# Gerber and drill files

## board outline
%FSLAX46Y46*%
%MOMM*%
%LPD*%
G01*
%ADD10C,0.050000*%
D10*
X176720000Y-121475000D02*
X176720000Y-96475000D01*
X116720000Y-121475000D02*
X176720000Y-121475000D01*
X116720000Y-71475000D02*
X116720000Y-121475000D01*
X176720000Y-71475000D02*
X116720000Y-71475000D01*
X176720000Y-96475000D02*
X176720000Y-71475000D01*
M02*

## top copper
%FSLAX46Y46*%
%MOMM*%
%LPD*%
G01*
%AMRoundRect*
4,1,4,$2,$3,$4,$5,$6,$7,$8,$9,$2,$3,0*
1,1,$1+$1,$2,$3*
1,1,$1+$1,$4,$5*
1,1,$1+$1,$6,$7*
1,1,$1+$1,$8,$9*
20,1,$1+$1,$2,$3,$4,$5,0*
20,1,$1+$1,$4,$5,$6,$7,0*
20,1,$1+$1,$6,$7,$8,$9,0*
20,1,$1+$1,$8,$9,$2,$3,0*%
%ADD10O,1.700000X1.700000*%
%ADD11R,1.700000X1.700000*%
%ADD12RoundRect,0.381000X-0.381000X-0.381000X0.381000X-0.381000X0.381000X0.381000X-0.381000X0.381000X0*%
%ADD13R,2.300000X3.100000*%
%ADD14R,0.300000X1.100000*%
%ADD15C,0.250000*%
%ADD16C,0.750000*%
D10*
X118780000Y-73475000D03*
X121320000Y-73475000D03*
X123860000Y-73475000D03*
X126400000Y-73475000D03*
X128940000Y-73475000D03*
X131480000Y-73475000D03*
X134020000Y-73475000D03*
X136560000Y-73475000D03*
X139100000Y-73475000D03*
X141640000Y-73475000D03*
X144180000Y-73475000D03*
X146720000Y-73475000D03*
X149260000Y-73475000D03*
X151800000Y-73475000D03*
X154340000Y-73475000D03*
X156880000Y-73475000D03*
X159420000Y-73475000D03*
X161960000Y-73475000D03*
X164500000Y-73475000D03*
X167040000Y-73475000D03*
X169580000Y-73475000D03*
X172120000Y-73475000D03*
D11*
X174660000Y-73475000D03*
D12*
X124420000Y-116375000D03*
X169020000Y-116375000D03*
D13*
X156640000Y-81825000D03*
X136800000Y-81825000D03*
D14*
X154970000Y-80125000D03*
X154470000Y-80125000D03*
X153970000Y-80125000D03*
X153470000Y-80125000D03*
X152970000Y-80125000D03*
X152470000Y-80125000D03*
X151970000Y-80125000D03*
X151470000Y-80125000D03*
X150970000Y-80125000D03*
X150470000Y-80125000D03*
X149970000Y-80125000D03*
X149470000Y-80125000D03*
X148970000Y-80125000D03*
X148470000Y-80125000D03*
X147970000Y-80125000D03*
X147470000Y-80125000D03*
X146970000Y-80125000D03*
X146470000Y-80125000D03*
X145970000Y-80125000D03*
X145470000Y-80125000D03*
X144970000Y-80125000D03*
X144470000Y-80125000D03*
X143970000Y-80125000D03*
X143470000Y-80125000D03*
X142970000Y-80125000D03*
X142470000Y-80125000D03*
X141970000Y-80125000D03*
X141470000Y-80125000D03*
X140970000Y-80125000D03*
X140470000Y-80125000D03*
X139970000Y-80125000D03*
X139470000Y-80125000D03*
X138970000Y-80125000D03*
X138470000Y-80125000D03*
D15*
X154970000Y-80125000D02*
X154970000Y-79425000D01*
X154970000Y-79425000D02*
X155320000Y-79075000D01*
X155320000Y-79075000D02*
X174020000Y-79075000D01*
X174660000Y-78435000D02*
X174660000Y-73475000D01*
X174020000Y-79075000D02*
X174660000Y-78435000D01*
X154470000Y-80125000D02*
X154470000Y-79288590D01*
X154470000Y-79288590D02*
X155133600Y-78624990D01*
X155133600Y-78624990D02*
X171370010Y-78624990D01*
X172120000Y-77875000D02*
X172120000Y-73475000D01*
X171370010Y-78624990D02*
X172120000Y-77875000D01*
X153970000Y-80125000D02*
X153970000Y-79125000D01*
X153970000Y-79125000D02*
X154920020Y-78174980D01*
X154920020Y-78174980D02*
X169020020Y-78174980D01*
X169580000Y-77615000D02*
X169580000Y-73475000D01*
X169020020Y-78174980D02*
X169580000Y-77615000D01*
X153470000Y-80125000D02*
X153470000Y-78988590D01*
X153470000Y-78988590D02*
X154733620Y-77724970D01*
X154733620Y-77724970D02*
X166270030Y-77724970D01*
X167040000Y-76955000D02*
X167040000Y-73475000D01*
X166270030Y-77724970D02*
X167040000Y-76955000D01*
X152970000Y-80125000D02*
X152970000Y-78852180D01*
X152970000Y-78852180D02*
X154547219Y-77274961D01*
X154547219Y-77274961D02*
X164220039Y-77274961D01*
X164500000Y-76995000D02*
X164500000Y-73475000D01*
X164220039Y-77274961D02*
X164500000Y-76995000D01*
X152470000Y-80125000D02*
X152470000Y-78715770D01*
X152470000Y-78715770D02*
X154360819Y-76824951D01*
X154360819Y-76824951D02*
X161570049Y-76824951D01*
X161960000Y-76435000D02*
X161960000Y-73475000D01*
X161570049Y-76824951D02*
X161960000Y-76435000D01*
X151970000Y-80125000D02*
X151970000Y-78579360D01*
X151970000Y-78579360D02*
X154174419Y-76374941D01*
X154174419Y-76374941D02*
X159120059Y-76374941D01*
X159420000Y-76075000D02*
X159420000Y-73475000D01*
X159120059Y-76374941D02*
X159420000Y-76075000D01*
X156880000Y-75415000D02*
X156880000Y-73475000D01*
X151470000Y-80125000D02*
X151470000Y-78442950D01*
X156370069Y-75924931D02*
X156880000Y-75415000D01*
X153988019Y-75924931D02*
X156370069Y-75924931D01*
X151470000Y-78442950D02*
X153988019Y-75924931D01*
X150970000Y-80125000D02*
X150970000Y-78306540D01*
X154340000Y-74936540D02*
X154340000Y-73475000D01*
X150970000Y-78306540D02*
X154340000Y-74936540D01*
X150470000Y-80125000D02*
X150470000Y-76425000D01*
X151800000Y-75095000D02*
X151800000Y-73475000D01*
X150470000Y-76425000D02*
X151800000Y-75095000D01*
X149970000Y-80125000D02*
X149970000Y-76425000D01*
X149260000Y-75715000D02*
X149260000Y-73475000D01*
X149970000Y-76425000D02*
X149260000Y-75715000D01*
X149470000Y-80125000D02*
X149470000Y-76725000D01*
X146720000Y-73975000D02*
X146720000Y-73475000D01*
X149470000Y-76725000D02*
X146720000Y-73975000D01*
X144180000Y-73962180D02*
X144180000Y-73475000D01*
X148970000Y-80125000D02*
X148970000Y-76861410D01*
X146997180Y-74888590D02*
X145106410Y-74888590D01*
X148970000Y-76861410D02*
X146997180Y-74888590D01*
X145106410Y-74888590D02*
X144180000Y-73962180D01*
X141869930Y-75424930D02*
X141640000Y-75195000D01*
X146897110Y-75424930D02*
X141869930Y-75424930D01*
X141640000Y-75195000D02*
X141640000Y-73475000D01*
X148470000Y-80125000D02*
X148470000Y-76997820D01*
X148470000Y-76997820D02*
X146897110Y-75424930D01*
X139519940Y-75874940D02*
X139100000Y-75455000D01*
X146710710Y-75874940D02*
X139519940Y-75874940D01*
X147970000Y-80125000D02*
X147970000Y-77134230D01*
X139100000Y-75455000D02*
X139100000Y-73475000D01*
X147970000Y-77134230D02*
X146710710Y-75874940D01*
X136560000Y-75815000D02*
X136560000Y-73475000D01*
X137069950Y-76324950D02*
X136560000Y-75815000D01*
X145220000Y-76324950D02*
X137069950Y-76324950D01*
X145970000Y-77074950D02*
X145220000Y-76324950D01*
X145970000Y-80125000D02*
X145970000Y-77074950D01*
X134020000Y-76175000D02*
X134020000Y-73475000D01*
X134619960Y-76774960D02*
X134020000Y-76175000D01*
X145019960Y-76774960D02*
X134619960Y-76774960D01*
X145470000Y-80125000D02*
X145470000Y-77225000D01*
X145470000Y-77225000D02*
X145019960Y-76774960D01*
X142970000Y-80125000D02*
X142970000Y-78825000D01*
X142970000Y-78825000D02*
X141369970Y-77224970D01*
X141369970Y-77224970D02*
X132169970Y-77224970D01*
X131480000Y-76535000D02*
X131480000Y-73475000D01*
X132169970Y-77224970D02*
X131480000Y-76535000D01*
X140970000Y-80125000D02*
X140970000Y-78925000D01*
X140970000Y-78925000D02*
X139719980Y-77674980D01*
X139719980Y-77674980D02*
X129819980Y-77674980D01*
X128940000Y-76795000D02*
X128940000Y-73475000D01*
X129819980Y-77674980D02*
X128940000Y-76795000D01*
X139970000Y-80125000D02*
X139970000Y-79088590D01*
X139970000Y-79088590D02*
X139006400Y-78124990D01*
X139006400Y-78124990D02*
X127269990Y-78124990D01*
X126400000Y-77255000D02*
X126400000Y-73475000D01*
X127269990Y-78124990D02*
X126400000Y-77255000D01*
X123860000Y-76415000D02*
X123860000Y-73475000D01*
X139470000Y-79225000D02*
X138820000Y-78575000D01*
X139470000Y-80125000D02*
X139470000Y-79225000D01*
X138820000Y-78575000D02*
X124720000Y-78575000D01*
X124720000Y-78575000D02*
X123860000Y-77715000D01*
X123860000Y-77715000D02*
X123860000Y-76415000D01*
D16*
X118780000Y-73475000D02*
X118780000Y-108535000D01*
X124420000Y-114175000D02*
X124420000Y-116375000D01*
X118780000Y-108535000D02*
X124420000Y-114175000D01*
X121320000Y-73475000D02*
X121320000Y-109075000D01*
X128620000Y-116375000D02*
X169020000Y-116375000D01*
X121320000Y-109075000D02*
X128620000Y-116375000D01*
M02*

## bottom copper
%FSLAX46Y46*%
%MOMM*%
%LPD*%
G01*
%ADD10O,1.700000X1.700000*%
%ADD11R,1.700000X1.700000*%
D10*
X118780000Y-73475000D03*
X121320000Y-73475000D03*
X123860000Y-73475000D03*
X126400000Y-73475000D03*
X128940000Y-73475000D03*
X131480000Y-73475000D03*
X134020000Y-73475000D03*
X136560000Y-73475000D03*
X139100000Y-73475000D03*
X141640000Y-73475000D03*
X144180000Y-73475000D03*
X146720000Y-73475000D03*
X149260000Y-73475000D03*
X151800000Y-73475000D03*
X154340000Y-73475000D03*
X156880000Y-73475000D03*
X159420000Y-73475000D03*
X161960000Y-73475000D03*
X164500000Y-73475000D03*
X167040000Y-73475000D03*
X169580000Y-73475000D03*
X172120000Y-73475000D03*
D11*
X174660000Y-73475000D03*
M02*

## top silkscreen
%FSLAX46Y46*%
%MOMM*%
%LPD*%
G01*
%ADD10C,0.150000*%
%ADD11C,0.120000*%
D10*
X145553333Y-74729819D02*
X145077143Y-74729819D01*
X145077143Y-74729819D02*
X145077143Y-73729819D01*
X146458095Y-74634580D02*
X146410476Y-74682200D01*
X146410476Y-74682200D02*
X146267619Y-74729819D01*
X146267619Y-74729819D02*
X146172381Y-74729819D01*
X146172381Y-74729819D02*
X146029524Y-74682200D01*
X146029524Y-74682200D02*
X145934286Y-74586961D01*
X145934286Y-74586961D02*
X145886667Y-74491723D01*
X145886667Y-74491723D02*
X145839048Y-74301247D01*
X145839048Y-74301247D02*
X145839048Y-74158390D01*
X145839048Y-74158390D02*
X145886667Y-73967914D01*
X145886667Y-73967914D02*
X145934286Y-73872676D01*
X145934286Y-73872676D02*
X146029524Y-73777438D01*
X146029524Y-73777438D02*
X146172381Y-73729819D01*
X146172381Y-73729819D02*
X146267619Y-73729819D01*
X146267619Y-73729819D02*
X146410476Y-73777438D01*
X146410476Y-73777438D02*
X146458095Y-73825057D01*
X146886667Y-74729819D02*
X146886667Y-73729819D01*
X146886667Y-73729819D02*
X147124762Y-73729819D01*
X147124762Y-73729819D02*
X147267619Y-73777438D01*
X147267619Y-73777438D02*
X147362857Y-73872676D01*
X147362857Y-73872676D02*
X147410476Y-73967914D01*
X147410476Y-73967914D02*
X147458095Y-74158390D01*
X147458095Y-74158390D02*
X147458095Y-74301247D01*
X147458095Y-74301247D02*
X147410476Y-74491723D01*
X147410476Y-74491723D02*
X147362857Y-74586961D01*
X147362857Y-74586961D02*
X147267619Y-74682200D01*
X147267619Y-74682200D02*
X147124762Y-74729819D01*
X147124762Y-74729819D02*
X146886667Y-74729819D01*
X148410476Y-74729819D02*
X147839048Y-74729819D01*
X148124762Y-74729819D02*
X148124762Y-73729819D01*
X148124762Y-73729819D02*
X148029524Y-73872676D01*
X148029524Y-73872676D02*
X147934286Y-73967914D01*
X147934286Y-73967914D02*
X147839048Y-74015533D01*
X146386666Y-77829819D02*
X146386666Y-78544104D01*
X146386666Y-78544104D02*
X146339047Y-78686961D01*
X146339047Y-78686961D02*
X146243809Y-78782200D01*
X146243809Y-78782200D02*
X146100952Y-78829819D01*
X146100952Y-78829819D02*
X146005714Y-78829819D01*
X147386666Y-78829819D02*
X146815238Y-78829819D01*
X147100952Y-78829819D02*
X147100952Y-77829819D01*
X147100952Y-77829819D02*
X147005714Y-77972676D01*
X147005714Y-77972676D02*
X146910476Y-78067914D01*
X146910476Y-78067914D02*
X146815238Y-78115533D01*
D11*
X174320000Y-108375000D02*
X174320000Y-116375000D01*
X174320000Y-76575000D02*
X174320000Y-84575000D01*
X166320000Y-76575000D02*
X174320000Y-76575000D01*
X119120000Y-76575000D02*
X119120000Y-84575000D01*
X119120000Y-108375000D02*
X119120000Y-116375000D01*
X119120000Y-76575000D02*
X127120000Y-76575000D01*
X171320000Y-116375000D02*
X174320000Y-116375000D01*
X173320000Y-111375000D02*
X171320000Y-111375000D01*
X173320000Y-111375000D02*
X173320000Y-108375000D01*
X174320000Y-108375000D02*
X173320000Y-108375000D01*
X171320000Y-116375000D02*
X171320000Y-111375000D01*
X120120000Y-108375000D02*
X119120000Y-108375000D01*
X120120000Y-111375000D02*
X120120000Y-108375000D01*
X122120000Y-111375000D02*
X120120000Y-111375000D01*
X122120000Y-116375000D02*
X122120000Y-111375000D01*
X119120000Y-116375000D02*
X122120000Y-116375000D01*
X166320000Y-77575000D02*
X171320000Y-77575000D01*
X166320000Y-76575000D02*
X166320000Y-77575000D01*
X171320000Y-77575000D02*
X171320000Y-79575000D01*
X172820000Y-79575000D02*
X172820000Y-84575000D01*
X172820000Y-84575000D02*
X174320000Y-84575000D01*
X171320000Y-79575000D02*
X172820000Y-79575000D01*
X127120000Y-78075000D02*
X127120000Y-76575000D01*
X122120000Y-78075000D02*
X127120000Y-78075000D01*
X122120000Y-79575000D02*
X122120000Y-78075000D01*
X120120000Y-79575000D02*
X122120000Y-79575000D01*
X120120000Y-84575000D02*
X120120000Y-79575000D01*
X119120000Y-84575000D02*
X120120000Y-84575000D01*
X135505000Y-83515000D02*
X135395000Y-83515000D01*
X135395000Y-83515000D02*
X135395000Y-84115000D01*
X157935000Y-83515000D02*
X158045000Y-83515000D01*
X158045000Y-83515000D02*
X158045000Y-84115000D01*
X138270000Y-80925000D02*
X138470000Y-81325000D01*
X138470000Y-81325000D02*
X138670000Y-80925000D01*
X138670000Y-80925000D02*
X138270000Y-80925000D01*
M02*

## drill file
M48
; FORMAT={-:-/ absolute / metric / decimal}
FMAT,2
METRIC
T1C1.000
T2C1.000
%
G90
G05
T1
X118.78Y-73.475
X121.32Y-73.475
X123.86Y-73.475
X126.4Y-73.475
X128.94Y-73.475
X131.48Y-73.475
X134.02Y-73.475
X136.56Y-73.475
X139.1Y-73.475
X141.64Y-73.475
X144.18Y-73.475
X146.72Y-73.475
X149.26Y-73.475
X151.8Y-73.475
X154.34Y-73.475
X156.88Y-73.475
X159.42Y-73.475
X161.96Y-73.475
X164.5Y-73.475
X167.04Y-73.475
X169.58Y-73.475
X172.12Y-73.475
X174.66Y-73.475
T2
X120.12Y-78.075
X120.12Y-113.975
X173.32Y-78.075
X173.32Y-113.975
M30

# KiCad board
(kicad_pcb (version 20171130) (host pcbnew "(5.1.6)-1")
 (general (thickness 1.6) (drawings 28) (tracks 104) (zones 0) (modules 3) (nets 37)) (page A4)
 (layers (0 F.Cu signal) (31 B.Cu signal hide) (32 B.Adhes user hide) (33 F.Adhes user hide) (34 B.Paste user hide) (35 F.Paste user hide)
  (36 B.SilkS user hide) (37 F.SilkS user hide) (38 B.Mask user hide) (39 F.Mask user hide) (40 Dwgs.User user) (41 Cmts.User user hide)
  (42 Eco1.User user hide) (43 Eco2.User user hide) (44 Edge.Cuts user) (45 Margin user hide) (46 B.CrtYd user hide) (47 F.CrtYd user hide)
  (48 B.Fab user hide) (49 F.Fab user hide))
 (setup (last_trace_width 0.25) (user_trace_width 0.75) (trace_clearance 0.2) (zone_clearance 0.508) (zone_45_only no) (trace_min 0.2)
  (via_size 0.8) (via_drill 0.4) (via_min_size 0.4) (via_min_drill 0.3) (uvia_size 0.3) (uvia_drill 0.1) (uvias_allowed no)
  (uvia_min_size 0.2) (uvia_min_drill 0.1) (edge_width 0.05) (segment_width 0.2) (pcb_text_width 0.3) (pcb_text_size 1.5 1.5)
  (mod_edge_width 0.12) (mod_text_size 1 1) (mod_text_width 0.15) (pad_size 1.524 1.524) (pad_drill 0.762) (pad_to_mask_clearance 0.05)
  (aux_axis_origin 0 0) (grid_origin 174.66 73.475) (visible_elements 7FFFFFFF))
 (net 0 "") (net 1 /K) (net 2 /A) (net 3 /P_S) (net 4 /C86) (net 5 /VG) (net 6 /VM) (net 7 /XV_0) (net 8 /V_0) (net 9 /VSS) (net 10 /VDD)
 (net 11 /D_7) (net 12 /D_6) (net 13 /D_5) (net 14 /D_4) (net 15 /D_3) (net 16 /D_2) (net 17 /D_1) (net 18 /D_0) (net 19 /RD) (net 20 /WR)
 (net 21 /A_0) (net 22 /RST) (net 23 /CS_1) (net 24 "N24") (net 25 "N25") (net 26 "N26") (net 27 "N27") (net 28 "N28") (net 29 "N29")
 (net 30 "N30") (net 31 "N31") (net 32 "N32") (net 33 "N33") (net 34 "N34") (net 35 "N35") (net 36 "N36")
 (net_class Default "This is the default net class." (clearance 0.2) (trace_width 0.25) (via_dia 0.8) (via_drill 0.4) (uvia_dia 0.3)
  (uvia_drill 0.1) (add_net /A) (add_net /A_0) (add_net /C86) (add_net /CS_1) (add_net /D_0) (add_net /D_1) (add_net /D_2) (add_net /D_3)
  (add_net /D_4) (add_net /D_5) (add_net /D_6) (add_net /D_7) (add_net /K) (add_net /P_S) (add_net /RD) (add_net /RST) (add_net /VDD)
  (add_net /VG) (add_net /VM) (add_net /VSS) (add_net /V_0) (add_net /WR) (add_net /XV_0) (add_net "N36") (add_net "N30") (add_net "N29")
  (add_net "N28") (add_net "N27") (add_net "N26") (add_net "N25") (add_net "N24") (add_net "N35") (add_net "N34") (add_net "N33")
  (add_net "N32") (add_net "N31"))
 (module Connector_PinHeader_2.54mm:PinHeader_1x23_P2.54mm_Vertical (layer B.Cu) (at 174.66 73.475 90)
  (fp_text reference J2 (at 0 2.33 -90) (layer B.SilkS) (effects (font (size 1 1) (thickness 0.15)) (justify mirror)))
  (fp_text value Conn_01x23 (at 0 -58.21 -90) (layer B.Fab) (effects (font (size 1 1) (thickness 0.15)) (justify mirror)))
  (pad 23 thru_hole oval (at 0 -55.88 90) (size 1.7 1.7) (drill 1) (layers *.Cu *.Mask) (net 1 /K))
  (pad 22 thru_hole oval (at 0 -53.34 90) (size 1.7 1.7) (drill 1) (layers *.Cu *.Mask) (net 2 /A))
  (pad 21 thru_hole oval (at 0 -50.8 90) (size 1.7 1.7) (drill 1) (layers *.Cu *.Mask) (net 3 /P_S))
  (pad 20 thru_hole oval (at 0 -48.26 90) (size 1.7 1.7) (drill 1) (layers *.Cu *.Mask) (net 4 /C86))
  (pad 19 thru_hole oval (at 0 -45.72 90) (size 1.7 1.7) (drill 1) (layers *.Cu *.Mask) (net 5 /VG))
  (pad 18 thru_hole oval (at 0 -43.18 90) (size 1.7 1.7) (drill 1) (layers *.Cu *.Mask) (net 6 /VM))
  (pad 17 thru_hole oval (at 0 -40.64 90) (size 1.7 1.7) (drill 1) (layers *.Cu *.Mask) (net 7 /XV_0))
  (pad 16 thru_hole oval (at 0 -38.1 90) (size 1.7 1.7) (drill 1) (layers *.Cu *.Mask) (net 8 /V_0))
  (pad 15 thru_hole oval (at 0 -35.56 90) (size 1.7 1.7) (drill 1) (layers *.Cu *.Mask) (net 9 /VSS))
  (pad 14 thru_hole oval (at 0 -33.02 90) (size 1.7 1.7) (drill 1) (layers *.Cu *.Mask) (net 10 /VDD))
  (pad 13 thru_hole oval (at 0 -30.48 90) (size 1.7 1.7) (drill 1) (layers *.Cu *.Mask) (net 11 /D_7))
  (pad 12 thru_hole oval (at 0 -27.94 90) (size 1.7 1.7) (drill 1) (layers *.Cu *.Mask) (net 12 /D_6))
  (pad 11 thru_hole oval (at 0 -25.4 90) (size 1.7 1.7) (drill 1) (layers *.Cu *.Mask) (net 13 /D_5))
  (pad 10 thru_hole oval (at 0 -22.86 90) (size 1.7 1.7) (drill 1) (layers *.Cu *.Mask) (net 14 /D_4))
  (pad 9 thru_hole oval (at 0 -20.32 90) (size 1.7 1.7) (drill 1) (layers *.Cu *.Mask) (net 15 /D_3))
  (pad 8 thru_hole oval (at 0 -17.78 90) (size 1.7 1.7) (drill 1) (layers *.Cu *.Mask) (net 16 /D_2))
  (pad 7 thru_hole oval (at 0 -15.24 90) (size 1.7 1.7) (drill 1) (layers *.Cu *.Mask) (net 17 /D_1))
  (pad 6 thru_hole oval (at 0 -12.7 90) (size 1.7 1.7) (drill 1) (layers *.Cu *.Mask) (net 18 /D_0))
  (pad 5 thru_hole oval (at 0 -10.16 90) (size 1.7 1.7) (drill 1) (layers *.Cu *.Mask) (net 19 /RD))
  (pad 4 thru_hole oval (at 0 -7.62 90) (size 1.7 1.7) (drill 1) (layers *.Cu *.Mask) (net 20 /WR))
  (pad 3 thru_hole oval (at 0 -5.08 90) (size 1.7 1.7) (drill 1) (layers *.Cu *.Mask) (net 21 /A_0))
  (pad 2 thru_hole oval (at 0 -2.54 90) (size 1.7 1.7) (drill 1) (layers *.Cu *.Mask) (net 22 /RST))
  (pad 1 thru_hole rect (at 0 0 90) (size 1.7 1.7) (drill 1) (layers *.Cu *.Mask) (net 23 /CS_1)))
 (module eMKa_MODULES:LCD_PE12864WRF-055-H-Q (layer F.Cu) (at 146.72 96.475)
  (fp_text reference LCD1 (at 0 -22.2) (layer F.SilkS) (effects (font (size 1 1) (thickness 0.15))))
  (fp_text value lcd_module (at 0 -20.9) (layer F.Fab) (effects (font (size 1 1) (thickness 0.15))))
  (fp_line (start 27.6 11.9) (end 27.6 19.9) (layer F.SilkS) (width 0.12))
  (fp_line (start 27.6 -19.9) (end 27.6 -11.9) (layer F.SilkS) (width 0.12))
  (fp_line (start 19.6 -19.9) (end 27.6 -19.9) (layer F.SilkS) (width 0.12))
  (fp_line (start -27.6 -19.9) (end -27.6 -11.9) (layer F.SilkS) (width 0.12))
  (fp_line (start -27.6 11.9) (end -27.6 19.9) (layer F.SilkS) (width 0.12))
  (fp_line (start -27.6 -19.9) (end -19.6 -19.9) (layer F.SilkS) (width 0.12))
  (fp_line (start 24.6 19.9) (end 27.6 19.9) (layer F.SilkS) (width 0.12))
  (fp_line (start 26.6 14.9) (end 24.6 14.9) (layer F.SilkS) (width 0.12))
  (fp_line (start 26.6 14.9) (end 26.6 11.9) (layer F.SilkS) (width 0.12))
  (fp_line (start 27.6 11.9) (end 26.6 11.9) (layer F.SilkS) (width 0.12))
  (fp_line (start 24.6 19.9) (end 24.6 14.9) (layer F.SilkS) (width 0.12))
  (fp_line (start -26.6 11.9) (end -27.6 11.9) (layer F.SilkS) (width 0.12))
  (fp_line (start -26.6 14.9) (end -26.6 11.9) (layer F.SilkS) (width 0.12))
  (fp_line (start -24.6 14.9) (end -26.6 14.9) (layer F.SilkS) (width 0.12))
  (fp_line (start -24.6 19.9) (end -24.6 14.9) (layer F.SilkS) (width 0.12))
  (fp_line (start -27.6 19.9) (end -24.6 19.9) (layer F.SilkS) (width 0.12))
  (fp_line (start 19.6 -18.9) (end 24.6 -18.9) (layer F.SilkS) (width 0.12))
  (fp_line (start 19.6 -19.9) (end 19.6 -18.9) (layer F.SilkS) (width 0.12))
  (fp_line (start 24.6 -18.9) (end 24.6 -16.9) (layer F.SilkS) (width 0.12))
  (fp_line (start 26.1 -16.9) (end 26.1 -11.9) (layer F.SilkS) (width 0.12))
  (fp_line (start 26.1 -11.9) (end 27.6 -11.9) (layer F.SilkS) (width 0.12))
  (fp_line (start 24.6 -16.9) (end 26.1 -16.9) (layer F.SilkS) (width 0.12))
  (fp_line (start -19.6 -18.4) (end -19.6 -19.9) (layer F.SilkS) (width 0.12))
  (fp_line (start -24.6 -18.4) (end -19.6 -18.4) (layer F.SilkS) (width 0.12))
  (fp_line (start -24.6 -16.9) (end -24.6 -18.4) (layer F.SilkS) (width 0.12))
  (fp_line (start -26.6 -16.9) (end -24.6 -16.9) (layer F.SilkS) (width 0.12))
  (fp_line (start -26.6 -11.9) (end -26.6 -16.9) (layer F.SilkS) (width 0.12))
  (fp_line (start -27.6 -11.9) (end -26.6 -11.9) (layer F.SilkS) (width 0.12))
  (pad 1 smd roundrect (at -22.3 19.9) (size 1.524 1.524) (layers F.Cu F.Paste F.Mask) (roundrect_rratio 0.25) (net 1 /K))
  (pad 2 smd roundrect (at 22.3 19.9) (size 1.524 1.524) (layers F.Cu F.Paste F.Mask) (roundrect_rratio 0.25) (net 2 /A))
  (pad "" np_thru_hole circle (at -26.6 17.5) (size 1 1) (drill 1) (layers *.Cu *.Mask))
  (pad "" np_thru_hole circle (at 26.6 17.5) (size 1 1) (drill 1) (layers *.Cu *.Mask))
  (pad "" np_thru_hole circle (at 26.6 -18.4) (size 1 1) (drill 1) (layers *.Cu *.Mask))
  (pad "" np_thru_hole circle (at -26.6 -18.4) (size 1 1) (drill 1) (layers *.Cu *.Mask)))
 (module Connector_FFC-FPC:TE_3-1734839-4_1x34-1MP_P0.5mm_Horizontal (layer F.Cu) (at 146.72 81.475)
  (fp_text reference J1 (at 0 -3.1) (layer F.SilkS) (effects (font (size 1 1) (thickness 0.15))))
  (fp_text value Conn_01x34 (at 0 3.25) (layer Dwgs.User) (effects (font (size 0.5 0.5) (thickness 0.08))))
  (fp_line (start -11.215 2.04) (end -11.325 2.04) (layer F.SilkS) (width 0.12))
  (fp_line (start -11.325 2.04) (end -11.325 2.64) (layer F.SilkS) (width 0.12))
  (fp_line (start 11.215 2.04) (end 11.325 2.04) (layer F.SilkS) (width 0.12))
  (fp_line (start 11.325 2.04) (end 11.325 2.64) (layer F.SilkS) (width 0.12))
  (fp_line (start -8.45 -0.55) (end -8.25 -0.15) (layer F.SilkS) (width 0.12))
  (fp_line (start -8.25 -0.15) (end -8.05 -0.55) (layer F.SilkS) (width 0.12))
  (fp_line (start -8.05 -0.55) (end -8.45 -0.55) (layer F.SilkS) (width 0.12))
  (pad MP smd rect (at 9.92 0.35) (size 2.3 3.1) (layers F.Cu F.Paste F.Mask))
  (pad MP smd rect (at -9.92 0.35) (size 2.3 3.1) (layers F.Cu F.Paste F.Mask))
  (pad 34 smd rect (at 8.25 -1.35) (size 0.3 1.1) (layers F.Cu F.Paste F.Mask) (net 23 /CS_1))
  (pad 33 smd rect (at 7.75 -1.35) (size 0.3 1.1) (layers F.Cu F.Paste F.Mask) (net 22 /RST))
  (pad 32 smd rect (at 7.25 -1.35) (size 0.3 1.1) (layers F.Cu F.Paste F.Mask) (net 21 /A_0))
  (pad 31 smd rect (at 6.75 -1.35) (size 0.3 1.1) (layers F.Cu F.Paste F.Mask) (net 20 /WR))
  (pad 30 smd rect (at 6.25 -1.35) (size 0.3 1.1) (layers F.Cu F.Paste F.Mask) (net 19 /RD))
  (pad 29 smd rect (at 5.75 -1.35) (size 0.3 1.1) (layers F.Cu F.Paste F.Mask) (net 18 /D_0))
  (pad 28 smd rect (at 5.25 -1.35) (size 0.3 1.1) (layers F.Cu F.Paste F.Mask) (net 17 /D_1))
  (pad 27 smd rect (at 4.75 -1.35) (size 0.3 1.1) (layers F.Cu F.Paste F.Mask) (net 16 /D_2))
  (pad 26 smd rect (at 4.25 -1.35) (size 0.3 1.1) (layers F.Cu F.Paste F.Mask) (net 15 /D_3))
  (pad 25 smd rect (at 3.75 -1.35) (size 0.3 1.1) (layers F.Cu F.Paste F.Mask) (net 14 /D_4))
  (pad 24 smd rect (at 3.25 -1.35) (size 0.3 1.1) (layers F.Cu F.Paste F.Mask) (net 13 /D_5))
  (pad 23 smd rect (at 2.75 -1.35) (size 0.3 1.1) (layers F.Cu F.Paste F.Mask) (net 12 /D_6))
  (pad 22 smd rect (at 2.25 -1.35) (size 0.3 1.1) (layers F.Cu F.Paste F.Mask) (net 11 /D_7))
  (pad 21 smd rect (at 1.75 -1.35) (size 0.3 1.1) (layers F.Cu F.Paste F.Mask) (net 10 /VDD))
  (pad 20 smd rect (at 1.25 -1.35) (size 0.3 1.1) (layers F.Cu F.Paste F.Mask) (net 9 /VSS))
  (pad 19 smd rect (at 0.75 -1.35) (size 0.3 1.1) (layers F.Cu F.Paste F.Mask) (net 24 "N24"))
  (pad 18 smd rect (at 0.25 -1.35) (size 0.3 1.1) (layers F.Cu F.Paste F.Mask) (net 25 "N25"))
  (pad 17 smd rect (at -0.25 -1.35) (size 0.3 1.1) (layers F.Cu F.Paste F.Mask) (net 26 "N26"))
  (pad 16 smd rect (at -0.75 -1.35) (size 0.3 1.1) (layers F.Cu F.Paste F.Mask) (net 8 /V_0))
  (pad 15 smd rect (at -1.25 -1.35) (size 0.3 1.1) (layers F.Cu F.Paste F.Mask) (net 7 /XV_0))
  (pad 14 smd rect (at -1.75 -1.35) (size 0.3 1.1) (layers F.Cu F.Paste F.Mask) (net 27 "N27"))
  (pad 13 smd rect (at -2.25 -1.35) (size 0.3 1.1) (layers F.Cu F.Paste F.Mask) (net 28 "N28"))
  (pad 12 smd rect (at -2.75 -1.35) (size 0.3 1.1) (layers F.Cu F.Paste F.Mask) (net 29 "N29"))
  (pad 11 smd rect (at -3.25 -1.35) (size 0.3 1.1) (layers F.Cu F.Paste F.Mask) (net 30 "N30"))
  (pad 10 smd rect (at -3.75 -1.35) (size 0.3 1.1) (layers F.Cu F.Paste F.Mask) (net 6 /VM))
  (pad 9 smd rect (at -4.25 -1.35) (size 0.3 1.1) (layers F.Cu F.Paste F.Mask) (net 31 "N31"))
  (pad 8 smd rect (at -4.75 -1.35) (size 0.3 1.1) (layers F.Cu F.Paste F.Mask) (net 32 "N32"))
  (pad 7 smd rect (at -5.25 -1.35) (size 0.3 1.1) (layers F.Cu F.Paste F.Mask) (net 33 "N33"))
  (pad 6 smd rect (at -5.75 -1.35) (size 0.3 1.1) (layers F.Cu F.Paste F.Mask) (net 5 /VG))
  (pad 5 smd rect (at -6.25 -1.35) (size 0.3 1.1) (layers F.Cu F.Paste F.Mask) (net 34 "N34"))
  (pad 4 smd rect (at -6.75 -1.35) (size 0.3 1.1) (layers F.Cu F.Paste F.Mask) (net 4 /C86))
  (pad 3 smd rect (at -7.25 -1.35) (size 0.3 1.1) (layers F.Cu F.Paste F.Mask) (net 3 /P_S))
  (pad 2 smd rect (at -7.75 -1.35) (size 0.3 1.1) (layers F.Cu F.Paste F.Mask) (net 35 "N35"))
  (pad 1 smd rect (at -8.25 -1.35) (size 0.3 1.1) (layers F.Cu F.Paste F.Mask) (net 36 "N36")))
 (gr_line (start 176.72 121.475) (end 176.72 96.475) (layer Edge.Cuts) (width 0.05))
 (gr_line (start 116.72 121.475) (end 176.72 121.475) (layer Edge.Cuts) (width 0.05))
 (gr_line (start 116.72 71.475) (end 116.72 121.475) (layer Edge.Cuts) (width 0.05))
 (gr_line (start 176.72 71.475) (end 116.72 71.475) (layer Edge.Cuts) (width 0.05))
 (gr_line (start 176.72 96.475) (end 176.72 71.475) (layer Edge.Cuts) (width 0.05))
 (segment (start 154.97 80.125) (end 154.97 79.425) (width 0.25) (layer F.Cu) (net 23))
 (segment (start 154.97 79.425) (end 155.32 79.075) (width 0.25) (layer F.Cu) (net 23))
 (segment (start 155.32 79.075) (end 174.02 79.075) (width 0.25) (layer F.Cu) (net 23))
 (segment (start 174.66 78.435) (end 174.66 73.475) (width 0.25) (layer F.Cu) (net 23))
 (segment (start 174.02 79.075) (end 174.66 78.435) (width 0.25) (layer F.Cu) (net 23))
 (segment (start 154.47 80.125) (end 154.47 79.28859) (width 0.25) (layer F.Cu) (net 22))
 (segment (start 154.47 79.28859) (end 155.1336 78.62499) (width 0.25) (layer F.Cu) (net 22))
 (segment (start 155.1336 78.62499) (end 171.37001 78.62499) (width 0.25) (layer F.Cu) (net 22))
 (segment (start 172.12 77.875) (end 172.12 73.475) (width 0.25) (layer F.Cu) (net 22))
 (segment (start 171.37001 78.62499) (end 172.12 77.875) (width 0.25) (layer F.Cu) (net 22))
 (segment (start 153.97 80.125) (end 153.97 79.125) (width 0.25) (layer F.Cu) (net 21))
 (segment (start 153.97 79.125) (end 154.92002 78.17498) (width 0.25) (layer F.Cu) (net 21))
 (segment (start 154.92002 78.17498) (end 169.02002 78.17498) (width 0.25) (layer F.Cu) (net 21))
 (segment (start 169.58 77.615) (end 169.58 73.475) (width 0.25) (layer F.Cu) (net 21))
 (segment (start 169.02002 78.17498) (end 169.58 77.615) (width 0.25) (layer F.Cu) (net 21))
 (segment (start 153.47 80.125) (end 153.47 78.98859) (width 0.25) (layer F.Cu) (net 20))
 (segment (start 153.47 78.98859) (end 154.73362 77.72497) (width 0.25) (layer F.Cu) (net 20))
 (segment (start 154.73362 77.72497) (end 166.27003 77.72497) (width 0.25) (layer F.Cu) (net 20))
 (segment (start 167.04 76.955) (end 167.04 73.475) (width 0.25) (layer F.Cu) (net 20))
 (segment (start 166.27003 77.72497) (end 167.04 76.955) (width 0.25) (layer F.Cu) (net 20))
 (segment (start 152.97 80.125) (end 152.97 78.85218) (width 0.25) (layer F.Cu) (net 19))
 (segment (start 152.97 78.85218) (end 154.547219 77.274961) (width 0.25) (layer F.Cu) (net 19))
 (segment (start 154.547219 77.274961) (end 164.220039 77.274961) (width 0.25) (layer F.Cu) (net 19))
 (segment (start 164.5 76.995) (end 164.5 73.475) (width 0.25) (layer F.Cu) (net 19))
 (segment (start 164.220039 77.274961) (end 164.5 76.995) (width 0.25) (layer F.Cu) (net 19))
 (segment (start 152.47 80.125) (end 152.47 78.71577) (width 0.25) (layer F.Cu) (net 18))
 (segment (start 152.47 78.71577) (end 154.360819 76.824951) (width 0.25) (layer F.Cu) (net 18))
 (segment (start 154.360819 76.824951) (end 161.570049 76.824951) (width 0.25) (layer F.Cu) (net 18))
 (segment (start 161.96 76.435) (end 161.96 73.475) (width 0.25) (layer F.Cu) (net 18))
 (segment (start 161.570049 76.824951) (end 161.96 76.435) (width 0.25) (layer F.Cu) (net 18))
 (segment (start 151.97 80.125) (end 151.97 78.57936) (width 0.25) (layer F.Cu) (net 17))
 (segment (start 151.97 78.57936) (end 154.174419 76.374941) (width 0.25) (layer F.Cu) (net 17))
 (segment (start 154.174419 76.374941) (end 159.120059 76.374941) (width 0.25) (layer F.Cu) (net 17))
 (segment (start 159.42 76.075) (end 159.42 73.475) (width 0.25) (layer F.Cu) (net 17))
 (segment (start 159.120059 76.374941) (end 159.42 76.075) (width 0.25) (layer F.Cu) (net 17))
 (segment (start 156.88 75.415) (end 156.88 73.475) (width 0.25) (layer F.Cu) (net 16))
 (segment (start 151.47 80.125) (end 151.47 78.44295) (width 0.25) (layer F.Cu) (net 16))
 (segment (start 156.370069 75.924931) (end 156.88 75.415) (width 0.25) (layer F.Cu) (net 16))
 (segment (start 153.988019 75.924931) (end 156.370069 75.924931) (width 0.25) (layer F.Cu) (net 16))
 (segment (start 151.47 78.44295) (end 153.988019 75.924931) (width 0.25) (layer F.Cu) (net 16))
 (segment (start 150.97 80.125) (end 150.97 78.30654) (width 0.25) (layer F.Cu) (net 15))
 (segment (start 154.34 74.93654) (end 154.34 73.475) (width 0.25) (layer F.Cu) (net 15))
 (segment (start 150.97 78.30654) (end 154.34 74.93654) (width 0.25) (layer F.Cu) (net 15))
 (segment (start 150.47 80.125) (end 150.47 76.425) (width 0.25) (layer F.Cu) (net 14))
 (segment (start 151.8 75.095) (end 151.8 73.475) (width 0.25) (layer F.Cu) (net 14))
 (segment (start 150.47 76.425) (end 151.8 75.095) (width 0.25) (layer F.Cu) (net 14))
 (segment (start 149.97 80.125) (end 149.97 76.425) (width 0.25) (layer F.Cu) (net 13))
 (segment (start 149.26 75.715) (end 149.26 73.475) (width 0.25) (layer F.Cu) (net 13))
 (segment (start 149.97 76.425) (end 149.26 75.715) (width 0.25) (layer F.Cu) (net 13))
 (segment (start 149.47 80.125) (end 149.47 76.725) (width 0.25) (layer F.Cu) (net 12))
 (segment (start 146.72 73.975) (end 146.72 73.475) (width 0.25) (layer F.Cu) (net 12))
 (segment (start 149.47 76.725) (end 146.72 73.975) (width 0.25) (layer F.Cu) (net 12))
 (segment (start 144.18 73.96218) (end 144.18 73.475) (width 0.25) (layer F.Cu) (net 11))
 (segment (start 148.97 80.125) (end 148.97 76.86141) (width 0.25) (layer F.Cu) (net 11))
 (segment (start 146.99718 74.88859) (end 145.10641 74.88859) (width 0.25) (layer F.Cu) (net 11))
 (segment (start 148.97 76.86141) (end 146.99718 74.88859) (width 0.25) (layer F.Cu) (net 11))
 (segment (start 145.10641 74.88859) (end 144.18 73.96218) (width 0.25) (layer F.Cu) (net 11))
 (segment (start 141.86993 75.42493) (end 141.64 75.195) (width 0.25) (layer F.Cu) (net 10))
 (segment (start 146.89711 75.42493) (end 141.86993 75.42493) (width 0.25) (layer F.Cu) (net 10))
 (segment (start 141.64 75.195) (end 141.64 73.475) (width 0.25) (layer F.Cu) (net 10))
 (segment (start 148.47 80.125) (end 148.47 76.99782) (width 0.25) (layer F.Cu) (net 10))
 (segment (start 148.47 76.99782) (end 146.89711 75.42493) (width 0.25) (layer F.Cu) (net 10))
 (segment (start 139.51994 75.87494) (end 139.1 75.455) (width 0.25) (layer F.Cu) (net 9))
 (segment (start 146.71071 75.87494) (end 139.51994 75.87494) (width 0.25) (layer F.Cu) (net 9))
 (segment (start 147.97 80.125) (end 147.97 77.13423) (width 0.25) (layer F.Cu) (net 9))
 (segment (start 139.1 75.455) (end 139.1 73.475) (width 0.25) (layer F.Cu) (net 9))
 (segment (start 147.97 77.13423) (end 146.71071 75.87494) (width 0.25) (layer F.Cu) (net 9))
 (segment (start 136.56 75.815) (end 136.56 73.475) (width 0.25) (layer F.Cu) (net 8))
 (segment (start 137.06995 76.32495) (end 136.56 75.815) (width 0.25) (layer F.Cu) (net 8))
 (segment (start 145.22 76.32495) (end 137.06995 76.32495) (width 0.25) (layer F.Cu) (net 8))
 (segment (start 145.97 77.07495) (end 145.22 76.32495) (width 0.25) (layer F.Cu) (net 8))
 (segment (start 145.97 80.125) (end 145.97 77.07495) (width 0.25) (layer F.Cu) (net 8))
 (segment (start 134.02 76.175) (end 134.02 73.475) (width 0.25) (layer F.Cu) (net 7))
 (segment (start 134.61996 76.77496) (end 134.02 76.175) (width 0.25) (layer F.Cu) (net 7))
 (segment (start 145.01996 76.77496) (end 134.61996 76.77496) (width 0.25) (layer F.Cu) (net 7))
 (segment (start 145.47 80.125) (end 145.47 77.225) (width 0.25) (layer F.Cu) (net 7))
 (segment (start 145.47 77.225) (end 145.01996 76.77496) (width 0.25) (layer F.Cu) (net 7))
 (segment (start 142.97 80.125) (end 142.97 78.825) (width 0.25) (layer F.Cu) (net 6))
 (segment (start 142.97 78.825) (end 141.36997 77.22497) (width 0.25) (layer F.Cu) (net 6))
 (segment (start 141.36997 77.22497) (end 132.16997 77.22497) (width 0.25) (layer F.Cu) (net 6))
 (segment (start 131.48 76.535) (end 131.48 73.475) (width 0.25) (layer F.Cu) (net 6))
 (segment (start 132.16997 77.22497) (end 131.48 76.535) (width 0.25) (layer F.Cu) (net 6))
 (segment (start 140.97 80.125) (end 140.97 78.925) (width 0.25) (layer F.Cu) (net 5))
 (segment (start 140.97 78.925) (end 139.71998 77.67498) (width 0.25) (layer F.Cu) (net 5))
 (segment (start 139.71998 77.67498) (end 129.81998 77.67498) (width 0.25) (layer F.Cu) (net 5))
 (segment (start 128.94 76.795) (end 128.94 73.475) (width 0.25) (layer F.Cu) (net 5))
 (segment (start 129.81998 77.67498) (end 128.94 76.795) (width 0.25) (layer F.Cu) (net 5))
 (segment (start 139.97 80.125) (end 139.97 79.08859) (width 0.25) (layer F.Cu) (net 4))
 (segment (start 139.97 79.08859) (end 139.0064 78.12499) (width 0.25) (layer F.Cu) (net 4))
 (segment (start 139.0064 78.12499) (end 127.26999 78.12499) (width 0.25) (layer F.Cu) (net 4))
 (segment (start 126.4 77.255) (end 126.4 73.475) (width 0.25) (layer F.Cu) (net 4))
 (segment (start 127.26999 78.12499) (end 126.4 77.255) (width 0.25) (layer F.Cu) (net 4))
 (segment (start 123.86 76.415) (end 123.86 73.475) (width 0.25) (layer F.Cu) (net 3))
 (segment (start 139.47 79.225) (end 138.82 78.575) (width 0.25) (layer F.Cu) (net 3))
 (segment (start 139.47 80.125) (end 139.47 79.225) (width 0.25) (layer F.Cu) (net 3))
 (segment (start 138.82 78.575) (end 124.72 78.575) (width 0.25) (layer F.Cu) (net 3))
 (segment (start 124.72 78.575) (end 123.86 77.715) (width 0.25) (layer F.Cu) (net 3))
 (segment (start 123.86 77.715) (end 123.86 76.415) (width 0.25) (layer F.Cu) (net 3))
 (segment (start 118.78 73.475) (end 118.78 108.535) (width 0.75) (layer F.Cu) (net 1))
 (segment (start 124.42 114.175) (end 124.42 116.375) (width 0.75) (layer F.Cu) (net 1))
 (segment (start 118.78 108.535) (end 124.42 114.175) (width 0.75) (layer F.Cu) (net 1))
 (segment (start 121.32 73.475) (end 121.32 109.075) (width 0.75) (layer F.Cu) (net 2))
 (segment (start 128.62 116.375) (end 169.02 116.375) (width 0.75) (layer F.Cu) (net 2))
 (segment (start 121.32 109.075) (end 128.62 116.375) (width 0.75) (layer F.Cu) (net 2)))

